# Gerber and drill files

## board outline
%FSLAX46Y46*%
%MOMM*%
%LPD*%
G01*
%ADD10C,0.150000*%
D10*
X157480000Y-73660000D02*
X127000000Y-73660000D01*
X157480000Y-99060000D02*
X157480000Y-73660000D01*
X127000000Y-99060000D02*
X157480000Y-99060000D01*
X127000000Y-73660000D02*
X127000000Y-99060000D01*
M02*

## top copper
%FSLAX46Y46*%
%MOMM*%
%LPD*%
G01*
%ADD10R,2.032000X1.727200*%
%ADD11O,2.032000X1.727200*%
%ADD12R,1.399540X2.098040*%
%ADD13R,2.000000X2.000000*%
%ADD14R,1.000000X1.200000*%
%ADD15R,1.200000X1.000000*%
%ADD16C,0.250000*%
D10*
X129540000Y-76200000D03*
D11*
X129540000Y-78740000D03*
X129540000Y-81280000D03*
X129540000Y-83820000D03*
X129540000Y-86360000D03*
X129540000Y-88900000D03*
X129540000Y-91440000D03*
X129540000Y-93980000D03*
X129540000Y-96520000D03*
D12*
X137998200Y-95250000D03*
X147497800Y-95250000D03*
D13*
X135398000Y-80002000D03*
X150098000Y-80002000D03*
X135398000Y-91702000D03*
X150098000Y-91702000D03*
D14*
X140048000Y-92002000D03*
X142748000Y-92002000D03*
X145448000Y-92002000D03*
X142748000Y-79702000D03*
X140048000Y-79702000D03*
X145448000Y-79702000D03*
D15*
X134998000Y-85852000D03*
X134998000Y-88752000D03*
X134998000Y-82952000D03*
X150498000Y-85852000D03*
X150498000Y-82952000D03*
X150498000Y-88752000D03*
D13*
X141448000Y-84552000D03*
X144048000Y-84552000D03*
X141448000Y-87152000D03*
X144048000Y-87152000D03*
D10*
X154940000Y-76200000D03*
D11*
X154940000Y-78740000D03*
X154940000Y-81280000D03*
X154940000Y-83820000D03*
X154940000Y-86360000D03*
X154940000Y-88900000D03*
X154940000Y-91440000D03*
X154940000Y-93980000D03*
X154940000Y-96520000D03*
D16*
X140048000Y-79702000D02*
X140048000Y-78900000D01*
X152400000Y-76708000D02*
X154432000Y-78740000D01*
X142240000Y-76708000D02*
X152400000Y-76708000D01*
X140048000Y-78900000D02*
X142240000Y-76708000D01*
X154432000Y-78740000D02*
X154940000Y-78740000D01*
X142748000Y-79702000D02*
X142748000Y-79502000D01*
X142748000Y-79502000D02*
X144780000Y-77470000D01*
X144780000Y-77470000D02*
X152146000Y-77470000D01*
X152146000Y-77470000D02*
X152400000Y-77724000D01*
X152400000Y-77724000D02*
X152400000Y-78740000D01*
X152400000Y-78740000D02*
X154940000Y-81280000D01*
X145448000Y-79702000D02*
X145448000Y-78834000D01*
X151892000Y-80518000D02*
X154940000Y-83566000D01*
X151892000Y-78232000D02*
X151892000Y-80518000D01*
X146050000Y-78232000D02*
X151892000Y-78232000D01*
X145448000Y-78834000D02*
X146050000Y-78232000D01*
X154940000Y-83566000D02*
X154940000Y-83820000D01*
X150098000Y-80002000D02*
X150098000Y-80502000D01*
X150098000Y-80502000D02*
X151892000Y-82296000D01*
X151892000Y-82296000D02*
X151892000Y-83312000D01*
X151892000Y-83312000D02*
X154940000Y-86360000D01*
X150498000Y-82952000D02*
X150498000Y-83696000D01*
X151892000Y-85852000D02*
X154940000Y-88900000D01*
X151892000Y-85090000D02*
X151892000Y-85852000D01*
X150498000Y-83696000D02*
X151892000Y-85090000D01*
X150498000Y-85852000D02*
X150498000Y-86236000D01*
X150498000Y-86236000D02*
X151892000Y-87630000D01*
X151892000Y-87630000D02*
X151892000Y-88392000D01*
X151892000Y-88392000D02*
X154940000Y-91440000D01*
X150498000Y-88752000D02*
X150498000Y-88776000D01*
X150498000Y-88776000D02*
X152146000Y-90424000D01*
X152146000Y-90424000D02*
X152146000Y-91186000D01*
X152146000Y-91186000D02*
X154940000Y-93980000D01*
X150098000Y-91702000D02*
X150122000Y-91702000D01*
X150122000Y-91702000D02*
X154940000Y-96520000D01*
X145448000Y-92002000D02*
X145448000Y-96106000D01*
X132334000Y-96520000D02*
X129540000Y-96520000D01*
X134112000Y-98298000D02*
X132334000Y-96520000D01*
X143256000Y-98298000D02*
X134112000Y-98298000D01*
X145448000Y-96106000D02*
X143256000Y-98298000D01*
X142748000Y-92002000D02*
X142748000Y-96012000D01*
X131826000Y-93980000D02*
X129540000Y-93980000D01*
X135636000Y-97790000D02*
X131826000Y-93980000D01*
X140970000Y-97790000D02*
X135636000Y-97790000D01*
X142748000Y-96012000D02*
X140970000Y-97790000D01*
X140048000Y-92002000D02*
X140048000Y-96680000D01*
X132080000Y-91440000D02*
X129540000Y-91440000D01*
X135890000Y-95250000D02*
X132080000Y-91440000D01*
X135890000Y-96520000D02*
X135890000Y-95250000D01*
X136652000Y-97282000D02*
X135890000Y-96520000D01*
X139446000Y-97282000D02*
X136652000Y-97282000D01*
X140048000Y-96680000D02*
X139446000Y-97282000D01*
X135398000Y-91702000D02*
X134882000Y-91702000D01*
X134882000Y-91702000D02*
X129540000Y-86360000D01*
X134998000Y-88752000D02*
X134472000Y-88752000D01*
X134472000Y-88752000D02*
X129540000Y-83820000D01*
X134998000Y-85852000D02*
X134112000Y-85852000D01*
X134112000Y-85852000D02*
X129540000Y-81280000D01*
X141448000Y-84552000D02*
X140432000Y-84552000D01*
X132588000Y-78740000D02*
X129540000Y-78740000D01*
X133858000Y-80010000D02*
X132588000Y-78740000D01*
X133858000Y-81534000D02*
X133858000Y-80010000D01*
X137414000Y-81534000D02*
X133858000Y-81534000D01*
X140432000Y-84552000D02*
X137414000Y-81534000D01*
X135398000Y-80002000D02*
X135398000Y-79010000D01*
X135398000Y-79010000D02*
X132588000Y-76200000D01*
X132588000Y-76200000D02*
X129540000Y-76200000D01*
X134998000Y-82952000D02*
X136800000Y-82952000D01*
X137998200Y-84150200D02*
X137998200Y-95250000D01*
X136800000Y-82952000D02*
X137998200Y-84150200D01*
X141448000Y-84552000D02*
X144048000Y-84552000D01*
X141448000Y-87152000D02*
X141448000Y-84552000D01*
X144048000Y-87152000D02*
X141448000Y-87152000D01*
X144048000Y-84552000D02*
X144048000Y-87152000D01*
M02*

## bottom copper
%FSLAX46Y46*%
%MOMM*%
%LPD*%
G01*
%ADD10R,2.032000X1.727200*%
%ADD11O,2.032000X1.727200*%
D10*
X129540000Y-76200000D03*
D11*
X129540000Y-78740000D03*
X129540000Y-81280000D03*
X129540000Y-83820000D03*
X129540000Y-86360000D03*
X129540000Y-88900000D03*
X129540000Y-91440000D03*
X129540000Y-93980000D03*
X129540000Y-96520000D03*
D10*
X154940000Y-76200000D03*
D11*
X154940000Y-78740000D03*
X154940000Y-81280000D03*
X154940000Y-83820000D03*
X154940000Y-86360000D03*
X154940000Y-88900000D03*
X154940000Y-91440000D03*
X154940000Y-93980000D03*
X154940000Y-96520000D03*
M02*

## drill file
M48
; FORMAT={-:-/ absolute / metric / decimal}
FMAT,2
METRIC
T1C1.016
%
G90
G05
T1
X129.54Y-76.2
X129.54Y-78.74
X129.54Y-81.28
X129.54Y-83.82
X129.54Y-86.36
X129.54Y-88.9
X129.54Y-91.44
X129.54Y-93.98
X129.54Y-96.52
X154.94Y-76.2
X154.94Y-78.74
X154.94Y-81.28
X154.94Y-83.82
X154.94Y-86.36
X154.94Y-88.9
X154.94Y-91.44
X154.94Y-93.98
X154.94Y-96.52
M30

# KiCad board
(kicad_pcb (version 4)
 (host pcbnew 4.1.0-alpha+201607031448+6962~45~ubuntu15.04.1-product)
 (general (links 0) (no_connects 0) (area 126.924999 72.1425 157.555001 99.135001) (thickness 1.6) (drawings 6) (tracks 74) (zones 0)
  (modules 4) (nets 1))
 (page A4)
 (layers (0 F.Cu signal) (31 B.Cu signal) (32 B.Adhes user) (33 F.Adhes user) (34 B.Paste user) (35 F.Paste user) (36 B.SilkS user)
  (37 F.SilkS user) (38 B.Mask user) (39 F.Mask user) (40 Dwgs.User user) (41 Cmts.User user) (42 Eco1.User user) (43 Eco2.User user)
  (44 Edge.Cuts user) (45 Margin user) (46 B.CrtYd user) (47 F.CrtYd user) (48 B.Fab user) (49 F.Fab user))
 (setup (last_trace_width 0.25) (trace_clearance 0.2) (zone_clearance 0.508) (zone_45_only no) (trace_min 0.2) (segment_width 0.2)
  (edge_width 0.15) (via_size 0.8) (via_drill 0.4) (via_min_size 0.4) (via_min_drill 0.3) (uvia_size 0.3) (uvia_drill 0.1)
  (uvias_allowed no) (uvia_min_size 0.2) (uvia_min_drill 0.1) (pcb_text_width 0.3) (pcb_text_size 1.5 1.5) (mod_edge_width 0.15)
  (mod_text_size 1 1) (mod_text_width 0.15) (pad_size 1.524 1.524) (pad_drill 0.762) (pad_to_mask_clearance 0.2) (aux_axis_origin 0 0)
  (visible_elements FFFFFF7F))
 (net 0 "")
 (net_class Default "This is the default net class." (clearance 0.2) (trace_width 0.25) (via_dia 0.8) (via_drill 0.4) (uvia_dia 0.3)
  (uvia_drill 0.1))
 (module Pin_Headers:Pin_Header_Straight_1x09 (layer F.Cu) (at 129.54 76.2)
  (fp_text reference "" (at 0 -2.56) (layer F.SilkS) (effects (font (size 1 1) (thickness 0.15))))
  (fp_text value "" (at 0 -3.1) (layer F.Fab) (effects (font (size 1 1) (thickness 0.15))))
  (pad 1 thru_hole rect (at 0 0) (size 2.032 1.7272) (drill 1.016) (layers *.Cu *.Mask F.SilkS))
  (pad 2 thru_hole oval (at 0 2.54) (size 2.032 1.7272) (drill 1.016) (layers *.Cu *.Mask F.SilkS))
  (pad 3 thru_hole oval (at 0 5.08) (size 2.032 1.7272) (drill 1.016) (layers *.Cu *.Mask F.SilkS))
  (pad 4 thru_hole oval (at 0 7.62) (size 2.032 1.7272) (drill 1.016) (layers *.Cu *.Mask F.SilkS))
  (pad 5 thru_hole oval (at 0 10.16) (size 2.032 1.7272) (drill 1.016) (layers *.Cu *.Mask F.SilkS))
  (pad 6 thru_hole oval (at 0 12.7) (size 2.032 1.7272) (drill 1.016) (layers *.Cu *.Mask F.SilkS))
  (pad 7 thru_hole oval (at 0 15.24) (size 2.032 1.7272) (drill 1.016) (layers *.Cu *.Mask F.SilkS))
  (pad 8 thru_hole oval (at 0 17.78) (size 2.032 1.7272) (drill 1.016) (layers *.Cu *.Mask F.SilkS))
  (pad 9 thru_hole oval (at 0 20.32) (size 2.032 1.7272) (drill 1.016) (layers *.Cu *.Mask F.SilkS)))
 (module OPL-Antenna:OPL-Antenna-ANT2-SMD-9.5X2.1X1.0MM (layer F.Cu) (at 142.748 95.25)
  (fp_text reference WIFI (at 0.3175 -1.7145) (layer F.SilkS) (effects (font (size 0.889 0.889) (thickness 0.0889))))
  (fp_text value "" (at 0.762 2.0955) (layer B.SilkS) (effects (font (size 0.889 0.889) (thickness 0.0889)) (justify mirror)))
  (pad 1 smd rect (at -4.7498 0) (size 1.39954 2.09804) (layers F.Cu F.Paste F.Mask))
  (pad 2 smd rect (at 4.7498 0) (size 1.39954 2.09804) (layers F.Cu F.Paste F.Mask)))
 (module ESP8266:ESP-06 (layer F.Cu) (at 142.748 85.852)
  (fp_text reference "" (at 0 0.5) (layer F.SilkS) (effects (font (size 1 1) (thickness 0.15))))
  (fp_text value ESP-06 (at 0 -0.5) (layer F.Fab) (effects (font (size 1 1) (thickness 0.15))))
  (pad G smd rect (at -7.35 -5.85) (size 2 2) (layers F.Cu F.Paste F.Mask))
  (pad G smd rect (at 7.35 -5.85) (size 2 2) (layers F.Cu F.Paste F.Mask))
  (pad G smd rect (at -7.35 5.85) (size 2 2) (layers F.Cu F.Paste F.Mask))
  (pad G smd rect (at 7.35 5.85) (size 2 2) (layers F.Cu F.Paste F.Mask))
  (pad GP14 smd rect (at -2.7 6.15) (size 1 1.2) (layers F.Cu F.Paste F.Mask))
  (pad GP13 smd rect (at 0 6.15) (size 1 1.2) (layers F.Cu F.Paste F.Mask))
  (pad GP12 smd rect (at 2.7 6.15) (size 1 1.2) (layers F.Cu F.Paste F.Mask))
  (pad TX smd rect (at 0 -6.15) (size 1 1.2) (layers F.Cu F.Paste F.Mask))
  (pad GP16 smd rect (at -2.7 -6.15) (size 1 1.2) (layers F.Cu F.Paste F.Mask))
  (pad RX smd rect (at 2.7 -6.15) (size 1 1.2) (layers F.Cu F.Paste F.Mask))
  (pad 3.3 smd rect (at -7.75 0) (size 1.2 1) (layers F.Cu F.Paste F.Mask))
  (pad CHPD smd rect (at -7.75 2.9) (size 1.2 1) (layers F.Cu F.Paste F.Mask))
  (pad ANT smd rect (at -7.75 -2.9) (size 1.2 1) (layers F.Cu F.Paste F.Mask))
  (pad GP2 smd rect (at 7.75 0) (size 1.2 1) (layers F.Cu F.Paste F.Mask))
  (pad GP0 smd rect (at 7.75 -2.9) (size 1.2 1) (layers F.Cu F.Paste F.Mask))
  (pad GP15 smd rect (at 7.75 2.9) (size 1.2 1) (layers F.Cu F.Paste F.Mask))
  (pad Gx smd rect (at -1.3 -1.3) (size 2 2) (layers F.Cu F.Paste F.Mask))
  (pad Gx smd rect (at 1.3 -1.3) (size 2 2) (layers F.Cu F.Paste F.Mask))
  (pad Gx smd rect (at -1.3 1.3) (size 2 2) (layers F.Cu F.Paste F.Mask))
  (pad Gx smd rect (at 1.3 1.3) (size 2 2) (layers F.Cu F.Paste F.Mask)))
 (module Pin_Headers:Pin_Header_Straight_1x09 (layer F.Cu) (at 154.94 76.2)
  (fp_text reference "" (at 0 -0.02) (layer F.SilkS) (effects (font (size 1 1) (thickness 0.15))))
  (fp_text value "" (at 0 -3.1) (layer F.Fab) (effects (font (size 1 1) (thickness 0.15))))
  (pad 1 thru_hole rect (at 0 0) (size 2.032 1.7272) (drill 1.016) (layers *.Cu *.Mask F.SilkS))
  (pad 2 thru_hole oval (at 0 2.54) (size 2.032 1.7272) (drill 1.016) (layers *.Cu *.Mask F.SilkS))
  (pad 3 thru_hole oval (at 0 5.08) (size 2.032 1.7272) (drill 1.016) (layers *.Cu *.Mask F.SilkS))
  (pad 4 thru_hole oval (at 0 7.62) (size 2.032 1.7272) (drill 1.016) (layers *.Cu *.Mask F.SilkS))
  (pad 5 thru_hole oval (at 0 10.16) (size 2.032 1.7272) (drill 1.016) (layers *.Cu *.Mask F.SilkS))
  (pad 6 thru_hole oval (at 0 12.7) (size 2.032 1.7272) (drill 1.016) (layers *.Cu *.Mask F.SilkS))
  (pad 7 thru_hole oval (at 0 15.24) (size 2.032 1.7272) (drill 1.016) (layers *.Cu *.Mask F.SilkS))
  (pad 8 thru_hole oval (at 0 17.78) (size 2.032 1.7272) (drill 1.016) (layers *.Cu *.Mask F.SilkS))
  (pad 9 thru_hole oval (at 0 20.32) (size 2.032 1.7272) (drill 1.016) (layers *.Cu *.Mask F.SilkS)))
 (gr_line (start 157.48 73.66) (end 127 73.66) (angle 90) (layer Edge.Cuts) (width 0.15))
 (gr_line (start 157.48 99.06) (end 157.48 73.66) (angle 90) (layer Edge.Cuts) (width 0.15))
 (gr_line (start 127 99.06) (end 157.48 99.06) (angle 90) (layer Edge.Cuts) (width 0.15))
 (gr_line (start 127 73.66) (end 127 99.06) (angle 90) (layer Edge.Cuts) (width 0.15))
 (segment (start 140.048 79.702) (end 140.048 78.9) (width 0.25) (layer F.Cu) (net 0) (status 400000))
 (segment (start 152.4 76.708) (end 154.432 78.74) (width 0.25) (layer F.Cu) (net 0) (status 800000))
 (segment (start 142.24 76.708) (end 152.4 76.708) (width 0.25) (layer F.Cu) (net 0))
 (segment (start 140.048 78.9) (end 142.24 76.708) (width 0.25) (layer F.Cu) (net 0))
 (segment (start 154.432 78.74) (end 154.94 78.74) (width 0.25) (layer F.Cu) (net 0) (status C00000))
 (segment (start 142.748 79.702) (end 142.748 79.502) (width 0.25) (layer F.Cu) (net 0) (status C00000))
 (segment (start 142.748 79.502) (end 144.78 77.47) (width 0.25) (layer F.Cu) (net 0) (status 400000))
 (segment (start 144.78 77.47) (end 152.146 77.47) (width 0.25) (layer F.Cu) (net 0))
 (segment (start 152.146 77.47) (end 152.4 77.724) (width 0.25) (layer F.Cu) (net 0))
 (segment (start 152.4 77.724) (end 152.4 78.74) (width 0.25) (layer F.Cu) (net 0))
 (segment (start 152.4 78.74) (end 154.94 81.28) (width 0.25) (layer F.Cu) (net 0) (status 800000))
 (segment (start 145.448 79.702) (end 145.448 78.834) (width 0.25) (layer F.Cu) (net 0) (status 400000))
 (segment (start 151.892 80.518) (end 154.94 83.566) (width 0.25) (layer F.Cu) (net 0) (status 800000))
 (segment (start 151.892 78.232) (end 151.892 80.518) (width 0.25) (layer F.Cu) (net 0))
 (segment (start 146.05 78.232) (end 151.892 78.232) (width 0.25) (layer F.Cu) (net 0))
 (segment (start 145.448 78.834) (end 146.05 78.232) (width 0.25) (layer F.Cu) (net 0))
 (segment (start 154.94 83.566) (end 154.94 83.82) (width 0.25) (layer F.Cu) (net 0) (status C00000))
 (segment (start 150.098 80.002) (end 150.098 80.502) (width 0.25) (layer F.Cu) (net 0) (status C00000))
 (segment (start 150.098 80.502) (end 151.892 82.296) (width 0.25) (layer F.Cu) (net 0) (status 400000))
 (segment (start 151.892 82.296) (end 151.892 83.312) (width 0.25) (layer F.Cu) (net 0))
 (segment (start 151.892 83.312) (end 154.94 86.36) (width 0.25) (layer F.Cu) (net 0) (status 800000))
 (segment (start 150.498 82.952) (end 150.498 83.696) (width 0.25) (layer F.Cu) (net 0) (status 400000))
 (segment (start 151.892 85.852) (end 154.94 88.9) (width 0.25) (layer F.Cu) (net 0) (status 800000))
 (segment (start 151.892 85.09) (end 151.892 85.852) (width 0.25) (layer F.Cu) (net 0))
 (segment (start 150.498 83.696) (end 151.892 85.09) (width 0.25) (layer F.Cu) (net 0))
 (segment (start 150.498 85.852) (end 150.498 86.236) (width 0.25) (layer F.Cu) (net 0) (status C00000))
 (segment (start 150.498 86.236) (end 151.892 87.63) (width 0.25) (layer F.Cu) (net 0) (status 400000))
 (segment (start 151.892 87.63) (end 151.892 88.392) (width 0.25) (layer F.Cu) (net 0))
 (segment (start 151.892 88.392) (end 154.94 91.44) (width 0.25) (layer F.Cu) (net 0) (status 800000))
 (segment (start 150.498 88.752) (end 150.498 88.776) (width 0.25) (layer F.Cu) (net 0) (status C00000))
 (segment (start 150.498 88.776) (end 152.146 90.424) (width 0.25) (layer F.Cu) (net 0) (status 400000))
 (segment (start 152.146 90.424) (end 152.146 91.186) (width 0.25) (layer F.Cu) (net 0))
 (segment (start 152.146 91.186) (end 154.94 93.98) (width 0.25) (layer F.Cu) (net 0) (status 800000))
 (segment (start 150.098 91.702) (end 150.122 91.702) (width 0.25) (layer F.Cu) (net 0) (status C00000))
 (segment (start 150.122 91.702) (end 154.94 96.52) (width 0.25) (layer F.Cu) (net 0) (status C00000))
 (segment (start 145.448 92.002) (end 145.448 96.106) (width 0.25) (layer F.Cu) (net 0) (status 400000))
 (segment (start 132.334 96.52) (end 129.54 96.52) (width 0.25) (layer F.Cu) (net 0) (status 800000))
 (segment (start 134.112 98.298) (end 132.334 96.52) (width 0.25) (layer F.Cu) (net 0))
 (segment (start 143.256 98.298) (end 134.112 98.298) (width 0.25) (layer F.Cu) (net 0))
 (segment (start 145.448 96.106) (end 143.256 98.298) (width 0.25) (layer F.Cu) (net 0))
 (segment (start 142.748 92.002) (end 142.748 96.012) (width 0.25) (layer F.Cu) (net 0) (status 400000))
 (segment (start 131.826 93.98) (end 129.54 93.98) (width 0.25) (layer F.Cu) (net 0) (status 800000))
 (segment (start 135.636 97.79) (end 131.826 93.98) (width 0.25) (layer F.Cu) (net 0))
 (segment (start 140.97 97.79) (end 135.636 97.79) (width 0.25) (layer F.Cu) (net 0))
 (segment (start 142.748 96.012) (end 140.97 97.79) (width 0.25) (layer F.Cu) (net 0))
 (segment (start 140.048 92.002) (end 140.048 96.68) (width 0.25) (layer F.Cu) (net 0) (status 400000))
 (segment (start 132.08 91.44) (end 129.54 91.44) (width 0.25) (layer F.Cu) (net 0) (status 800000))
 (segment (start 135.89 95.25) (end 132.08 91.44) (width 0.25) (layer F.Cu) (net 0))
 (segment (start 135.89 96.52) (end 135.89 95.25) (width 0.25) (layer F.Cu) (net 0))
 (segment (start 136.652 97.282) (end 135.89 96.52) (width 0.25) (layer F.Cu) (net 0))
 (segment (start 139.446 97.282) (end 136.652 97.282) (width 0.25) (layer F.Cu) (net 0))
 (segment (start 140.048 96.68) (end 139.446 97.282) (width 0.25) (layer F.Cu) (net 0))
 (segment (start 135.398 91.702) (end 134.882 91.702) (width 0.25) (layer F.Cu) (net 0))
 (segment (start 134.882 91.702) (end 129.54 86.36) (width 0.25) (layer F.Cu) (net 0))
 (segment (start 134.998 88.752) (end 134.472 88.752) (width 0.25) (layer F.Cu) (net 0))
 (segment (start 134.472 88.752) (end 129.54 83.82) (width 0.25) (layer F.Cu) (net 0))
 (segment (start 134.998 85.852) (end 134.112 85.852) (width 0.25) (layer F.Cu) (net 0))
 (segment (start 134.112 85.852) (end 129.54 81.28) (width 0.25) (layer F.Cu) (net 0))
 (segment (start 141.448 84.552) (end 140.432 84.552) (width 0.25) (layer F.Cu) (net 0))
 (segment (start 132.588 78.74) (end 129.54 78.74) (width 0.25) (layer F.Cu) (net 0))
 (segment (start 133.858 80.01) (end 132.588 78.74) (width 0.25) (layer F.Cu) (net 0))
 (segment (start 133.858 81.534) (end 133.858 80.01) (width 0.25) (layer F.Cu) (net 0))
 (segment (start 137.414 81.534) (end 133.858 81.534) (width 0.25) (layer F.Cu) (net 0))
 (segment (start 140.432 84.552) (end 137.414 81.534) (width 0.25) (layer F.Cu) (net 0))
 (segment (start 135.398 80.002) (end 135.398 79.01) (width 0.25) (layer F.Cu) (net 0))
 (segment (start 135.398 79.01) (end 132.588 76.2) (width 0.25) (layer F.Cu) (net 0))
 (segment (start 132.588 76.2) (end 129.54 76.2) (width 0.25) (layer F.Cu) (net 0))
 (segment (start 134.998 82.952) (end 136.8 82.952) (width 0.25) (layer F.Cu) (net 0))
 (segment (start 137.9982 84.1502) (end 137.9982 95.25) (width 0.25) (layer F.Cu) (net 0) (status 20))
 (segment (start 136.8 82.952) (end 137.9982 84.1502) (width 0.25) (layer F.Cu) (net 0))
 (segment (start 141.448 84.552) (end 144.048 84.552) (width 0.25) (layer F.Cu) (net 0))
 (segment (start 141.448 87.152) (end 141.448 84.552) (width 0.25) (layer F.Cu) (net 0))
 (segment (start 144.048 87.152) (end 141.448 87.152) (width 0.25) (layer F.Cu) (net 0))
 (segment (start 144.048 84.552) (end 144.048 87.152) (width 0.25) (layer F.Cu) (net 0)))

